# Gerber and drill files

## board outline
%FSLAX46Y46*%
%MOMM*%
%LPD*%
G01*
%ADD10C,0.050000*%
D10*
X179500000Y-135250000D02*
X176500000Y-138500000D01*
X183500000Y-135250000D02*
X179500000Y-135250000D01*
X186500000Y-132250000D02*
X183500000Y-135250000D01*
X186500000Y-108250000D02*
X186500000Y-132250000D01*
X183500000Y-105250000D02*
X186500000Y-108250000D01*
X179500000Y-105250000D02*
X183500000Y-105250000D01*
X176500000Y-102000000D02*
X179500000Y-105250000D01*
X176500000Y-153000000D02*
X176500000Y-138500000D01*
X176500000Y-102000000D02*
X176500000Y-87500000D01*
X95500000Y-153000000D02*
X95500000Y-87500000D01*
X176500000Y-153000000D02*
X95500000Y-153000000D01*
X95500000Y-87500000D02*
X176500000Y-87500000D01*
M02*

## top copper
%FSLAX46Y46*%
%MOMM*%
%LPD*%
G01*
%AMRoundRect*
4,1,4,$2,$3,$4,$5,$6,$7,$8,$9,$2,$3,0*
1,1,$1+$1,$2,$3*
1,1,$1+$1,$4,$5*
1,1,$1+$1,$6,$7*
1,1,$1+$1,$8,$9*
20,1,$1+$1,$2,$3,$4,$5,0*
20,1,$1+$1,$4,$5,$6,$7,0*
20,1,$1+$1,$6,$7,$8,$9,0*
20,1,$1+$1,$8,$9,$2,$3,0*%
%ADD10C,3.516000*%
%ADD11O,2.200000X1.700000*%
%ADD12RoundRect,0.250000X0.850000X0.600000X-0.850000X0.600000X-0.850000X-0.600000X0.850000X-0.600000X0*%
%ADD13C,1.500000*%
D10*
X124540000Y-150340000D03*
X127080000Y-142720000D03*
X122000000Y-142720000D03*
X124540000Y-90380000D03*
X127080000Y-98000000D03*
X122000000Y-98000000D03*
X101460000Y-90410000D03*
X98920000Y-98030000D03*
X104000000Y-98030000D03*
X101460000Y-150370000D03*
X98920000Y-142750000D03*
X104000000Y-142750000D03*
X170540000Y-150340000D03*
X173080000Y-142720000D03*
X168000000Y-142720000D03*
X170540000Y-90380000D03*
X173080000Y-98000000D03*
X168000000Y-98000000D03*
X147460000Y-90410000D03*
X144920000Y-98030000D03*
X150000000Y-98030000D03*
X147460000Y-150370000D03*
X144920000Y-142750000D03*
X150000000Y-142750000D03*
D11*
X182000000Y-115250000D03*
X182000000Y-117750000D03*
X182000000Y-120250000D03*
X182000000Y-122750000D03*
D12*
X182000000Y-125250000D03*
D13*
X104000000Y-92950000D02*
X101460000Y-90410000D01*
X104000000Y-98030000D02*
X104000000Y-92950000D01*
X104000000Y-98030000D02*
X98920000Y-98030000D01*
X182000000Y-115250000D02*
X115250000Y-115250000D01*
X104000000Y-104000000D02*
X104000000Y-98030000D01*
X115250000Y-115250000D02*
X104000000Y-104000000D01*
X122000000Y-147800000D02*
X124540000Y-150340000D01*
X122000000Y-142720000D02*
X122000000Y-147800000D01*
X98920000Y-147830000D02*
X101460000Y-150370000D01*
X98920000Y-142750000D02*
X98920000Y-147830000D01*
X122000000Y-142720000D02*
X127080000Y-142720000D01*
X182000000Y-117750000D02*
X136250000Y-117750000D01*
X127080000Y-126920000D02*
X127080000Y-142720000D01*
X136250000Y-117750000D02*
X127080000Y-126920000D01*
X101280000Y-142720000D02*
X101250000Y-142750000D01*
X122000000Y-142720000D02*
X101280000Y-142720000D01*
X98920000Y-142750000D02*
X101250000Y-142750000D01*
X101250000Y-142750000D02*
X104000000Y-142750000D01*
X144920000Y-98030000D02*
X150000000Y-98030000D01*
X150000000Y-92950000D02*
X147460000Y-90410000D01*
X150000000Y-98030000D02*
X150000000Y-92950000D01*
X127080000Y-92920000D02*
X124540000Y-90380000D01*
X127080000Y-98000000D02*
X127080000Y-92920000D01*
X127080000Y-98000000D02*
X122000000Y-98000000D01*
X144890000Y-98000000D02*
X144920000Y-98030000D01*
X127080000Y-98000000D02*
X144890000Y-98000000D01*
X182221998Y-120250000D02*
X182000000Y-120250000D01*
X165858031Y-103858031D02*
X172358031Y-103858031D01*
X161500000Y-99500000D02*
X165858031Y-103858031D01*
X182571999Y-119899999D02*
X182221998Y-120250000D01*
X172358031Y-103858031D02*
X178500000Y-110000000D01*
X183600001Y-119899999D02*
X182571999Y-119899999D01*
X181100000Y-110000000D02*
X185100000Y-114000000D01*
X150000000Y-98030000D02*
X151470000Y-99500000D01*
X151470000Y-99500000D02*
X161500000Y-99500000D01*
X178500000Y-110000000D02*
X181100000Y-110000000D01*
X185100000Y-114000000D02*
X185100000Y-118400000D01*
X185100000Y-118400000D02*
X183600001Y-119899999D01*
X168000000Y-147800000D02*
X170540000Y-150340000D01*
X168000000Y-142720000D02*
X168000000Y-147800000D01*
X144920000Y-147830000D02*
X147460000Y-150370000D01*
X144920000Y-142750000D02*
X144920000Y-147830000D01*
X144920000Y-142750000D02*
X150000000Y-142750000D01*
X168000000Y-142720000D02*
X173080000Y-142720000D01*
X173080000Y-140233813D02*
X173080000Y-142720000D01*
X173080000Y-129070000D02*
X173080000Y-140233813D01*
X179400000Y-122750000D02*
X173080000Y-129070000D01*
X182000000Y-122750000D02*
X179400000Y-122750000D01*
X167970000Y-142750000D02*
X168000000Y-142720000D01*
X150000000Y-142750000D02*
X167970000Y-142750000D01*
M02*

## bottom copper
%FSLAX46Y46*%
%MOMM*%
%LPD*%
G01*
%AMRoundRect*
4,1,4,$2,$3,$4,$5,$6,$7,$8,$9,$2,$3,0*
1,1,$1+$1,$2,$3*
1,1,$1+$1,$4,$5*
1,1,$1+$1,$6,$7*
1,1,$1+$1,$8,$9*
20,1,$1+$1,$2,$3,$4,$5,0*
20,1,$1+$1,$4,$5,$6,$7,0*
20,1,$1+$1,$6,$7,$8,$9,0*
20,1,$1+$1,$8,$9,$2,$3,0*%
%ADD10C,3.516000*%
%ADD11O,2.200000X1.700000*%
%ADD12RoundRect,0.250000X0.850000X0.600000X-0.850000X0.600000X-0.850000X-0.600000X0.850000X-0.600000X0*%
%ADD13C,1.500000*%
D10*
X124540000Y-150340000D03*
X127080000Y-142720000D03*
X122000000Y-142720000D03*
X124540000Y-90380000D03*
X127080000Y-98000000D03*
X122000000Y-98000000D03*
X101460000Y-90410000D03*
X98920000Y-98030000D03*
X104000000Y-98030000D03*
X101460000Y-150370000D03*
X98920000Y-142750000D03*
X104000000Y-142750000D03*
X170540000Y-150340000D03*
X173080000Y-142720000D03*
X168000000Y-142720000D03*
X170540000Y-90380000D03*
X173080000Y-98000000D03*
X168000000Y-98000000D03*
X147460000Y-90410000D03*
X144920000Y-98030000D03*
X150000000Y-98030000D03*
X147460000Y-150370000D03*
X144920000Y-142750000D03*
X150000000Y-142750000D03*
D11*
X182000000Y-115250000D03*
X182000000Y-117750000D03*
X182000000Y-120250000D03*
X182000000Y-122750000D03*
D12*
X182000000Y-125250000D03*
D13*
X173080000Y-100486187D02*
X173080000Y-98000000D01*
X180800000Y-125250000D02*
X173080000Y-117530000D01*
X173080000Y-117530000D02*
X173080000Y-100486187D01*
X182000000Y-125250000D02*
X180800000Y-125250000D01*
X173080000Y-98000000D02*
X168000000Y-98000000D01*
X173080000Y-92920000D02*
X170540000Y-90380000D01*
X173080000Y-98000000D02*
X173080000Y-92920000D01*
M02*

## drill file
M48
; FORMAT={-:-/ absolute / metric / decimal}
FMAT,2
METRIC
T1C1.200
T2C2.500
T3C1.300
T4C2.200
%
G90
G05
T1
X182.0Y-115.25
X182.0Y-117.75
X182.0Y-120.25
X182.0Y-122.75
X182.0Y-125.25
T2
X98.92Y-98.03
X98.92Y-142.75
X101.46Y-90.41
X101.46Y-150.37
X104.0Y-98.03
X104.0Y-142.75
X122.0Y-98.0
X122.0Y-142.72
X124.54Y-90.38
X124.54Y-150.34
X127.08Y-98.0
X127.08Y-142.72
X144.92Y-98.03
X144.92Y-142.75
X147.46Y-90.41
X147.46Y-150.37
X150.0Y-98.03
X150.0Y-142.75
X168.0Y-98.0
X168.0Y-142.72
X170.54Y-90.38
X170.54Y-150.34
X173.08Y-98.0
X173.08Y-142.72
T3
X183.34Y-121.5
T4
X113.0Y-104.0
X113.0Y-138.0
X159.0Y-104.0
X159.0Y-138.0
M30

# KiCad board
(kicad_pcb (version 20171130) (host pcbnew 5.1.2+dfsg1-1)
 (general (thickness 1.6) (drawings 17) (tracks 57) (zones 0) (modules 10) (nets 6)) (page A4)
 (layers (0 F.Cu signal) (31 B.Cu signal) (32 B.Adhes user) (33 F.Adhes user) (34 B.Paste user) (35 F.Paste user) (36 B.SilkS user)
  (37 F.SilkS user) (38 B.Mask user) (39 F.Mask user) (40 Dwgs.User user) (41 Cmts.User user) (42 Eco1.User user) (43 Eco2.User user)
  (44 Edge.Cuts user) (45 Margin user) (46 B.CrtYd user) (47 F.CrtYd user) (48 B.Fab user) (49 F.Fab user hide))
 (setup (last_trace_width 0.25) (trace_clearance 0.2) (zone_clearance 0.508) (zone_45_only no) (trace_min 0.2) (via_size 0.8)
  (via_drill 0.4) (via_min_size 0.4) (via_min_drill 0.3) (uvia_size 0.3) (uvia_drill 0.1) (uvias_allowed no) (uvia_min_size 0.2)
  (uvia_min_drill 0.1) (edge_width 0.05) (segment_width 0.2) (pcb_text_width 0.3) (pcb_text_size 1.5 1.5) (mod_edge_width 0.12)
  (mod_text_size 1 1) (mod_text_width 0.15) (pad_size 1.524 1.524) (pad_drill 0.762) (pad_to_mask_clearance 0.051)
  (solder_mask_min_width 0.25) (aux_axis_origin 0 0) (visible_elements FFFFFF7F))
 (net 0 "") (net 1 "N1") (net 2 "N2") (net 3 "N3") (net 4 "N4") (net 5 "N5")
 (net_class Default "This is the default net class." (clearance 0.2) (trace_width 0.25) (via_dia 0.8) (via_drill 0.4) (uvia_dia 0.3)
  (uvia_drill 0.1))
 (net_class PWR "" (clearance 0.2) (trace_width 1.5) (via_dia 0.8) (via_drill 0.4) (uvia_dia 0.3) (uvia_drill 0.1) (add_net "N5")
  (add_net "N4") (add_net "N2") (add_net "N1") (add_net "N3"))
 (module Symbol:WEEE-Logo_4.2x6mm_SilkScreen (layer F.Cu) (at 113 93)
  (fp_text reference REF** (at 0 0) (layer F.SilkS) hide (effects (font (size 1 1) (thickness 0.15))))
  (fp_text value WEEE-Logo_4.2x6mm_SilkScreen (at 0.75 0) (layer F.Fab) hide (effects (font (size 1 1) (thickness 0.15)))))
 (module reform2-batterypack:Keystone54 (layer F.Cu) (at 122 98)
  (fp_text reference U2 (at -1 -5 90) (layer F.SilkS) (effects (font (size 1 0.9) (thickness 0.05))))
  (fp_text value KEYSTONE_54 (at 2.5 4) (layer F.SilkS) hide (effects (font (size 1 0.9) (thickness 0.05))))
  (pad 6 thru_hole circle (at 2.54 52.34) (size 3.516 3.516) (drill 2.5) (layers *.Cu *.Mask) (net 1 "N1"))
  (pad 5 thru_hole circle (at 5.08 44.72) (size 3.516 3.516) (drill 2.5) (layers *.Cu *.Mask) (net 1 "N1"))
  (pad 4 thru_hole circle (at 0 44.72) (size 3.516 3.516) (drill 2.5) (layers *.Cu *.Mask) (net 1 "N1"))
  (pad 3 thru_hole circle (at 2.54 -7.62) (size 3.516 3.516) (drill 2.5) (layers *.Cu *.Mask) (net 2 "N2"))
  (pad 2 thru_hole circle (at 5.08 0) (size 3.516 3.516) (drill 2.5) (layers *.Cu *.Mask) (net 2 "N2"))
  (pad 1 thru_hole circle (at 0 0) (size 3.516 3.516) (drill 2.5) (layers *.Cu *.Mask) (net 2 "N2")))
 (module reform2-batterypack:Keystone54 (layer F.Cu) (at 104 142.75 180)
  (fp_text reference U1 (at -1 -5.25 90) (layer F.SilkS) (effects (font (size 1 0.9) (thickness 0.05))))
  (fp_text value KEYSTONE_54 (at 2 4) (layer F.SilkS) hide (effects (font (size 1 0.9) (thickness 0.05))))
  (pad 6 thru_hole circle (at 2.54 52.34 180) (size 3.516 3.516) (drill 2.5) (layers *.Cu *.Mask) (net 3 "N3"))
  (pad 5 thru_hole circle (at 5.08 44.72 180) (size 3.516 3.516) (drill 2.5) (layers *.Cu *.Mask) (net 3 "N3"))
  (pad 4 thru_hole circle (at 0 44.72 180) (size 3.516 3.516) (drill 2.5) (layers *.Cu *.Mask) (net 3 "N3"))
  (pad 3 thru_hole circle (at 2.54 -7.62 180) (size 3.516 3.516) (drill 2.5) (layers *.Cu *.Mask) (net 1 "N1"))
  (pad 2 thru_hole circle (at 5.08 0 180) (size 3.516 3.516) (drill 2.5) (layers *.Cu *.Mask) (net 1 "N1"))
  (pad 1 thru_hole circle (at 0 0 180) (size 3.516 3.516) (drill 2.5) (layers *.Cu *.Mask) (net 1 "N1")))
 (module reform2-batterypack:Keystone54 (layer F.Cu) (at 168 98)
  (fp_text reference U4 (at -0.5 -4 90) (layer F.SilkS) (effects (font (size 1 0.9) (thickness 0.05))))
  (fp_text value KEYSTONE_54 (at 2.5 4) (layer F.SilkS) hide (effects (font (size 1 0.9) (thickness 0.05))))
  (pad 6 thru_hole circle (at 2.54 52.34) (size 3.516 3.516) (drill 2.5) (layers *.Cu *.Mask) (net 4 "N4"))
  (pad 5 thru_hole circle (at 5.08 44.72) (size 3.516 3.516) (drill 2.5) (layers *.Cu *.Mask) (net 4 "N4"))
  (pad 4 thru_hole circle (at 0 44.72) (size 3.516 3.516) (drill 2.5) (layers *.Cu *.Mask) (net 4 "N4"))
  (pad 3 thru_hole circle (at 2.54 -7.62) (size 3.516 3.516) (drill 2.5) (layers *.Cu *.Mask) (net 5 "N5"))
  (pad 2 thru_hole circle (at 5.08 0) (size 3.516 3.516) (drill 2.5) (layers *.Cu *.Mask) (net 5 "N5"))
  (pad 1 thru_hole circle (at 0 0) (size 3.516 3.516) (drill 2.5) (layers *.Cu *.Mask) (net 5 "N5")))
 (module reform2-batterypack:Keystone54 (layer F.Cu) (at 150 142.75 180)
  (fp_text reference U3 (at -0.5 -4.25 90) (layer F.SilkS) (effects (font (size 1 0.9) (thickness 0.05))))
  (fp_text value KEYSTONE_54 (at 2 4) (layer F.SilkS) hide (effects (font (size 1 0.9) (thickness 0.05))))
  (pad 6 thru_hole circle (at 2.54 52.34 180) (size 3.516 3.516) (drill 2.5) (layers *.Cu *.Mask) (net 2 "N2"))
  (pad 5 thru_hole circle (at 5.08 44.72 180) (size 3.516 3.516) (drill 2.5) (layers *.Cu *.Mask) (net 2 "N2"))
  (pad 4 thru_hole circle (at 0 44.72 180) (size 3.516 3.516) (drill 2.5) (layers *.Cu *.Mask) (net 2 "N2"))
  (pad 3 thru_hole circle (at 2.54 -7.62 180) (size 3.516 3.516) (drill 2.5) (layers *.Cu *.Mask) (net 4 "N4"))
  (pad 2 thru_hole circle (at 5.08 0 180) (size 3.516 3.516) (drill 2.5) (layers *.Cu *.Mask) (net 4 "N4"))
  (pad 1 thru_hole circle (at 0 0 180) (size 3.516 3.516) (drill 2.5) (layers *.Cu *.Mask) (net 4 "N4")))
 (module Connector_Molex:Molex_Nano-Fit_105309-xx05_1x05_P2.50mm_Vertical (layer F.Cu) (at 182 125.25 180)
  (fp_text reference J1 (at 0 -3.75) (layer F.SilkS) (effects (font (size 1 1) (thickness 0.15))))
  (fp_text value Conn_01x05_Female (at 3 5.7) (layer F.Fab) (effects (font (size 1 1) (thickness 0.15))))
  (pad "" np_thru_hole circle (at -1.34 3.75 180) (size 1.3 1.3) (drill 1.3) (layers *.Cu *.Mask))
  (pad 5 thru_hole oval (at 0 10 180) (size 2.2 1.7) (drill 1.2) (layers *.Cu *.Mask) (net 3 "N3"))
  (pad 4 thru_hole oval (at 0 7.5 180) (size 2.2 1.7) (drill 1.2) (layers *.Cu *.Mask) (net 1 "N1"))
  (pad 3 thru_hole oval (at 0 5 180) (size 2.2 1.7) (drill 1.2) (layers *.Cu *.Mask) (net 2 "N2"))
  (pad 2 thru_hole oval (at 0 2.5 180) (size 2.2 1.7) (drill 1.2) (layers *.Cu *.Mask) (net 4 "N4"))
  (pad 1 thru_hole roundrect (at 0 0 180) (size 2.2 1.7) (drill 1.2) (layers *.Cu *.Mask) (roundrect_rratio 0.147059) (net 5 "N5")))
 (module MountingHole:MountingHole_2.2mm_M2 (layer F.Cu) (at 159 138)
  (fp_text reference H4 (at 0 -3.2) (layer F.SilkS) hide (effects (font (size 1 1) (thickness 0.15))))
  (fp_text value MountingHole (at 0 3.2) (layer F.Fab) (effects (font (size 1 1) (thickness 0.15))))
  (pad 1 np_thru_hole circle (at 0 0) (size 2.2 2.2) (drill 2.2) (layers *.Cu *.Mask)))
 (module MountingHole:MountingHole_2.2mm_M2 (layer F.Cu) (at 113 138)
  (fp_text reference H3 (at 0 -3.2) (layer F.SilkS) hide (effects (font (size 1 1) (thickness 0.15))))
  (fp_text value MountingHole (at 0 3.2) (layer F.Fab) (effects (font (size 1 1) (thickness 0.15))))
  (pad 1 np_thru_hole circle (at 0 0) (size 2.2 2.2) (drill 2.2) (layers *.Cu *.Mask)))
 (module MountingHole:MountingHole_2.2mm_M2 (layer F.Cu) (at 159 104)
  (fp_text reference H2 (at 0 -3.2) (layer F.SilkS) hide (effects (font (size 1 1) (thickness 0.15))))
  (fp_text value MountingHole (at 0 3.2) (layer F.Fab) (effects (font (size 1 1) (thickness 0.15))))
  (pad 1 np_thru_hole circle (at 0 0) (size 2.2 2.2) (drill 2.2) (layers *.Cu *.Mask)))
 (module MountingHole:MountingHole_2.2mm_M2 (layer F.Cu) (at 113 104)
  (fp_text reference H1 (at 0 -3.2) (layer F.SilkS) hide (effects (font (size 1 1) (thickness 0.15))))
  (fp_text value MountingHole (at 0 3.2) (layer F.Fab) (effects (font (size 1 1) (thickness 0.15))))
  (pad 1 np_thru_hole circle (at 0 0) (size 2.2 2.2) (drill 2.2) (layers *.Cu *.Mask)))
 (gr_line (start 179.5 135.25) (end 176.5 138.5) (layer Edge.Cuts) (width 0.05))
 (gr_line (start 183.5 135.25) (end 179.5 135.25) (layer Edge.Cuts) (width 0.05))
 (gr_line (start 186.5 132.25) (end 183.5 135.25) (layer Edge.Cuts) (width 0.05))
 (gr_line (start 186.5 108.25) (end 186.5 132.25) (layer Edge.Cuts) (width 0.05))
 (gr_line (start 183.5 105.25) (end 186.5 108.25) (layer Edge.Cuts) (width 0.05))
 (gr_line (start 179.5 105.25) (end 183.5 105.25) (layer Edge.Cuts) (width 0.05))
 (gr_line (start 176.5 102) (end 179.5 105.25) (layer Edge.Cuts) (width 0.05))
 (gr_line (start 176.5 153) (end 176.5 138.5) (layer Edge.Cuts) (width 0.05))
 (gr_line (start 176.5 102) (end 176.5 87.5) (layer Edge.Cuts) (width 0.05))
 (gr_line (start 95.5 153) (end 95.5 87.5) (layer Edge.Cuts) (width 0.05))
 (gr_line (start 176.5 153) (end 95.5 153) (layer Edge.Cuts) (width 0.05))
 (gr_line (start 95.5 87.5) (end 176.5 87.5) (layer Edge.Cuts) (width 0.05))
 (segment (start 104 92.95) (end 101.46 90.41) (width 1.5) (layer F.Cu) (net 3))
 (segment (start 104 98.03) (end 104 92.95) (width 1.5) (layer F.Cu) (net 3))
 (segment (start 104 98.03) (end 98.92 98.03) (width 1.5) (layer F.Cu) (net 3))
 (segment (start 182 115.25) (end 115.25 115.25) (width 1.5) (layer F.Cu) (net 3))
 (segment (start 104 104) (end 104 98.03) (width 1.5) (layer F.Cu) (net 3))
 (segment (start 115.25 115.25) (end 104 104) (width 1.5) (layer F.Cu) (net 3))
 (segment (start 122 147.8) (end 124.54 150.34) (width 1.5) (layer F.Cu) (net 1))
 (segment (start 122 142.72) (end 122 147.8) (width 1.5) (layer F.Cu) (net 1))
 (segment (start 98.92 147.83) (end 101.46 150.37) (width 1.5) (layer F.Cu) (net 1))
 (segment (start 98.92 142.75) (end 98.92 147.83) (width 1.5) (layer F.Cu) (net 1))
 (segment (start 122 142.72) (end 127.08 142.72) (width 1.5) (layer F.Cu) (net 1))
 (segment (start 182 117.75) (end 136.25 117.75) (width 1.5) (layer F.Cu) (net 1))
 (segment (start 127.08 126.92) (end 127.08 142.72) (width 1.5) (layer F.Cu) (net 1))
 (segment (start 136.25 117.75) (end 127.08 126.92) (width 1.5) (layer F.Cu) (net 1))
 (segment (start 101.28 142.72) (end 101.25 142.75) (width 1.5) (layer F.Cu) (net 1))
 (segment (start 122 142.72) (end 101.28 142.72) (width 1.5) (layer F.Cu) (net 1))
 (segment (start 98.92 142.75) (end 101.25 142.75) (width 1.5) (layer F.Cu) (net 1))
 (segment (start 101.25 142.75) (end 104 142.75) (width 1.5) (layer F.Cu) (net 1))
 (segment (start 144.92 98.03) (end 150 98.03) (width 1.5) (layer F.Cu) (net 2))
 (segment (start 150 92.95) (end 147.46 90.41) (width 1.5) (layer F.Cu) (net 2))
 (segment (start 150 98.03) (end 150 92.95) (width 1.5) (layer F.Cu) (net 2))
 (segment (start 127.08 92.92) (end 124.54 90.38) (width 1.5) (layer F.Cu) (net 2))
 (segment (start 127.08 98) (end 127.08 92.92) (width 1.5) (layer F.Cu) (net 2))
 (segment (start 127.08 98) (end 122 98) (width 1.5) (layer F.Cu) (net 2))
 (segment (start 144.89 98) (end 144.92 98.03) (width 1.5) (layer F.Cu) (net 2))
 (segment (start 127.08 98) (end 144.89 98) (width 1.5) (layer F.Cu) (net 2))
 (segment (start 182.221998 120.25) (end 182 120.25) (width 1.5) (layer F.Cu) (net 2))
 (segment (start 165.858031 103.858031) (end 172.358031 103.858031) (width 1.5) (layer F.Cu) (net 2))
 (segment (start 161.5 99.5) (end 165.858031 103.858031) (width 1.5) (layer F.Cu) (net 2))
 (segment (start 182.571999 119.899999) (end 182.221998 120.25) (width 1.5) (layer F.Cu) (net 2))
 (segment (start 172.358031 103.858031) (end 178.5 110) (width 1.5) (layer F.Cu) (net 2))
 (segment (start 183.600001 119.899999) (end 182.571999 119.899999) (width 1.5) (layer F.Cu) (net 2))
 (segment (start 181.1 110) (end 185.1 114) (width 1.5) (layer F.Cu) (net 2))
 (segment (start 150 98.03) (end 151.47 99.5) (width 1.5) (layer F.Cu) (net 2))
 (segment (start 151.47 99.5) (end 161.5 99.5) (width 1.5) (layer F.Cu) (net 2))
 (segment (start 178.5 110) (end 181.1 110) (width 1.5) (layer F.Cu) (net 2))
 (segment (start 185.1 114) (end 185.1 118.4) (width 1.5) (layer F.Cu) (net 2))
 (segment (start 185.1 118.4) (end 183.600001 119.899999) (width 1.5) (layer F.Cu) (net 2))
 (segment (start 168 147.8) (end 170.54 150.34) (width 1.5) (layer F.Cu) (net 4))
 (segment (start 168 142.72) (end 168 147.8) (width 1.5) (layer F.Cu) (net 4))
 (segment (start 144.92 147.83) (end 147.46 150.37) (width 1.5) (layer F.Cu) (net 4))
 (segment (start 144.92 142.75) (end 144.92 147.83) (width 1.5) (layer F.Cu) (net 4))
 (segment (start 144.92 142.75) (end 150 142.75) (width 1.5) (layer F.Cu) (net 4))
 (segment (start 168 142.72) (end 173.08 142.72) (width 1.5) (layer F.Cu) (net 4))
 (segment (start 173.08 140.233813) (end 173.08 142.72) (width 1.5) (layer F.Cu) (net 4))
 (segment (start 173.08 129.07) (end 173.08 140.233813) (width 1.5) (layer F.Cu) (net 4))
 (segment (start 179.4 122.75) (end 173.08 129.07) (width 1.5) (layer F.Cu) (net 4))
 (segment (start 182 122.75) (end 179.4 122.75) (width 1.5) (layer F.Cu) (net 4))
 (segment (start 167.97 142.75) (end 168 142.72) (width 1.5) (layer F.Cu) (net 4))
 (segment (start 150 142.75) (end 167.97 142.75) (width 1.5) (layer F.Cu) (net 4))
 (segment (start 173.08 100.486187) (end 173.08 98) (width 1.5) (layer B.Cu) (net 5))
 (segment (start 180.8 125.25) (end 173.08 117.53) (width 1.5) (layer B.Cu) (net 5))
 (segment (start 173.08 117.53) (end 173.08 100.486187) (width 1.5) (layer B.Cu) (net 5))
 (segment (start 182 125.25) (end 180.8 125.25) (width 1.5) (layer B.Cu) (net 5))
 (segment (start 173.08 98) (end 168 98) (width 1.5) (layer B.Cu) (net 5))
 (segment (start 173.08 92.92) (end 170.54 90.38) (width 1.5) (layer B.Cu) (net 5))
 (segment (start 173.08 98) (end 173.08 92.92) (width 1.5) (layer B.Cu) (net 5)))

